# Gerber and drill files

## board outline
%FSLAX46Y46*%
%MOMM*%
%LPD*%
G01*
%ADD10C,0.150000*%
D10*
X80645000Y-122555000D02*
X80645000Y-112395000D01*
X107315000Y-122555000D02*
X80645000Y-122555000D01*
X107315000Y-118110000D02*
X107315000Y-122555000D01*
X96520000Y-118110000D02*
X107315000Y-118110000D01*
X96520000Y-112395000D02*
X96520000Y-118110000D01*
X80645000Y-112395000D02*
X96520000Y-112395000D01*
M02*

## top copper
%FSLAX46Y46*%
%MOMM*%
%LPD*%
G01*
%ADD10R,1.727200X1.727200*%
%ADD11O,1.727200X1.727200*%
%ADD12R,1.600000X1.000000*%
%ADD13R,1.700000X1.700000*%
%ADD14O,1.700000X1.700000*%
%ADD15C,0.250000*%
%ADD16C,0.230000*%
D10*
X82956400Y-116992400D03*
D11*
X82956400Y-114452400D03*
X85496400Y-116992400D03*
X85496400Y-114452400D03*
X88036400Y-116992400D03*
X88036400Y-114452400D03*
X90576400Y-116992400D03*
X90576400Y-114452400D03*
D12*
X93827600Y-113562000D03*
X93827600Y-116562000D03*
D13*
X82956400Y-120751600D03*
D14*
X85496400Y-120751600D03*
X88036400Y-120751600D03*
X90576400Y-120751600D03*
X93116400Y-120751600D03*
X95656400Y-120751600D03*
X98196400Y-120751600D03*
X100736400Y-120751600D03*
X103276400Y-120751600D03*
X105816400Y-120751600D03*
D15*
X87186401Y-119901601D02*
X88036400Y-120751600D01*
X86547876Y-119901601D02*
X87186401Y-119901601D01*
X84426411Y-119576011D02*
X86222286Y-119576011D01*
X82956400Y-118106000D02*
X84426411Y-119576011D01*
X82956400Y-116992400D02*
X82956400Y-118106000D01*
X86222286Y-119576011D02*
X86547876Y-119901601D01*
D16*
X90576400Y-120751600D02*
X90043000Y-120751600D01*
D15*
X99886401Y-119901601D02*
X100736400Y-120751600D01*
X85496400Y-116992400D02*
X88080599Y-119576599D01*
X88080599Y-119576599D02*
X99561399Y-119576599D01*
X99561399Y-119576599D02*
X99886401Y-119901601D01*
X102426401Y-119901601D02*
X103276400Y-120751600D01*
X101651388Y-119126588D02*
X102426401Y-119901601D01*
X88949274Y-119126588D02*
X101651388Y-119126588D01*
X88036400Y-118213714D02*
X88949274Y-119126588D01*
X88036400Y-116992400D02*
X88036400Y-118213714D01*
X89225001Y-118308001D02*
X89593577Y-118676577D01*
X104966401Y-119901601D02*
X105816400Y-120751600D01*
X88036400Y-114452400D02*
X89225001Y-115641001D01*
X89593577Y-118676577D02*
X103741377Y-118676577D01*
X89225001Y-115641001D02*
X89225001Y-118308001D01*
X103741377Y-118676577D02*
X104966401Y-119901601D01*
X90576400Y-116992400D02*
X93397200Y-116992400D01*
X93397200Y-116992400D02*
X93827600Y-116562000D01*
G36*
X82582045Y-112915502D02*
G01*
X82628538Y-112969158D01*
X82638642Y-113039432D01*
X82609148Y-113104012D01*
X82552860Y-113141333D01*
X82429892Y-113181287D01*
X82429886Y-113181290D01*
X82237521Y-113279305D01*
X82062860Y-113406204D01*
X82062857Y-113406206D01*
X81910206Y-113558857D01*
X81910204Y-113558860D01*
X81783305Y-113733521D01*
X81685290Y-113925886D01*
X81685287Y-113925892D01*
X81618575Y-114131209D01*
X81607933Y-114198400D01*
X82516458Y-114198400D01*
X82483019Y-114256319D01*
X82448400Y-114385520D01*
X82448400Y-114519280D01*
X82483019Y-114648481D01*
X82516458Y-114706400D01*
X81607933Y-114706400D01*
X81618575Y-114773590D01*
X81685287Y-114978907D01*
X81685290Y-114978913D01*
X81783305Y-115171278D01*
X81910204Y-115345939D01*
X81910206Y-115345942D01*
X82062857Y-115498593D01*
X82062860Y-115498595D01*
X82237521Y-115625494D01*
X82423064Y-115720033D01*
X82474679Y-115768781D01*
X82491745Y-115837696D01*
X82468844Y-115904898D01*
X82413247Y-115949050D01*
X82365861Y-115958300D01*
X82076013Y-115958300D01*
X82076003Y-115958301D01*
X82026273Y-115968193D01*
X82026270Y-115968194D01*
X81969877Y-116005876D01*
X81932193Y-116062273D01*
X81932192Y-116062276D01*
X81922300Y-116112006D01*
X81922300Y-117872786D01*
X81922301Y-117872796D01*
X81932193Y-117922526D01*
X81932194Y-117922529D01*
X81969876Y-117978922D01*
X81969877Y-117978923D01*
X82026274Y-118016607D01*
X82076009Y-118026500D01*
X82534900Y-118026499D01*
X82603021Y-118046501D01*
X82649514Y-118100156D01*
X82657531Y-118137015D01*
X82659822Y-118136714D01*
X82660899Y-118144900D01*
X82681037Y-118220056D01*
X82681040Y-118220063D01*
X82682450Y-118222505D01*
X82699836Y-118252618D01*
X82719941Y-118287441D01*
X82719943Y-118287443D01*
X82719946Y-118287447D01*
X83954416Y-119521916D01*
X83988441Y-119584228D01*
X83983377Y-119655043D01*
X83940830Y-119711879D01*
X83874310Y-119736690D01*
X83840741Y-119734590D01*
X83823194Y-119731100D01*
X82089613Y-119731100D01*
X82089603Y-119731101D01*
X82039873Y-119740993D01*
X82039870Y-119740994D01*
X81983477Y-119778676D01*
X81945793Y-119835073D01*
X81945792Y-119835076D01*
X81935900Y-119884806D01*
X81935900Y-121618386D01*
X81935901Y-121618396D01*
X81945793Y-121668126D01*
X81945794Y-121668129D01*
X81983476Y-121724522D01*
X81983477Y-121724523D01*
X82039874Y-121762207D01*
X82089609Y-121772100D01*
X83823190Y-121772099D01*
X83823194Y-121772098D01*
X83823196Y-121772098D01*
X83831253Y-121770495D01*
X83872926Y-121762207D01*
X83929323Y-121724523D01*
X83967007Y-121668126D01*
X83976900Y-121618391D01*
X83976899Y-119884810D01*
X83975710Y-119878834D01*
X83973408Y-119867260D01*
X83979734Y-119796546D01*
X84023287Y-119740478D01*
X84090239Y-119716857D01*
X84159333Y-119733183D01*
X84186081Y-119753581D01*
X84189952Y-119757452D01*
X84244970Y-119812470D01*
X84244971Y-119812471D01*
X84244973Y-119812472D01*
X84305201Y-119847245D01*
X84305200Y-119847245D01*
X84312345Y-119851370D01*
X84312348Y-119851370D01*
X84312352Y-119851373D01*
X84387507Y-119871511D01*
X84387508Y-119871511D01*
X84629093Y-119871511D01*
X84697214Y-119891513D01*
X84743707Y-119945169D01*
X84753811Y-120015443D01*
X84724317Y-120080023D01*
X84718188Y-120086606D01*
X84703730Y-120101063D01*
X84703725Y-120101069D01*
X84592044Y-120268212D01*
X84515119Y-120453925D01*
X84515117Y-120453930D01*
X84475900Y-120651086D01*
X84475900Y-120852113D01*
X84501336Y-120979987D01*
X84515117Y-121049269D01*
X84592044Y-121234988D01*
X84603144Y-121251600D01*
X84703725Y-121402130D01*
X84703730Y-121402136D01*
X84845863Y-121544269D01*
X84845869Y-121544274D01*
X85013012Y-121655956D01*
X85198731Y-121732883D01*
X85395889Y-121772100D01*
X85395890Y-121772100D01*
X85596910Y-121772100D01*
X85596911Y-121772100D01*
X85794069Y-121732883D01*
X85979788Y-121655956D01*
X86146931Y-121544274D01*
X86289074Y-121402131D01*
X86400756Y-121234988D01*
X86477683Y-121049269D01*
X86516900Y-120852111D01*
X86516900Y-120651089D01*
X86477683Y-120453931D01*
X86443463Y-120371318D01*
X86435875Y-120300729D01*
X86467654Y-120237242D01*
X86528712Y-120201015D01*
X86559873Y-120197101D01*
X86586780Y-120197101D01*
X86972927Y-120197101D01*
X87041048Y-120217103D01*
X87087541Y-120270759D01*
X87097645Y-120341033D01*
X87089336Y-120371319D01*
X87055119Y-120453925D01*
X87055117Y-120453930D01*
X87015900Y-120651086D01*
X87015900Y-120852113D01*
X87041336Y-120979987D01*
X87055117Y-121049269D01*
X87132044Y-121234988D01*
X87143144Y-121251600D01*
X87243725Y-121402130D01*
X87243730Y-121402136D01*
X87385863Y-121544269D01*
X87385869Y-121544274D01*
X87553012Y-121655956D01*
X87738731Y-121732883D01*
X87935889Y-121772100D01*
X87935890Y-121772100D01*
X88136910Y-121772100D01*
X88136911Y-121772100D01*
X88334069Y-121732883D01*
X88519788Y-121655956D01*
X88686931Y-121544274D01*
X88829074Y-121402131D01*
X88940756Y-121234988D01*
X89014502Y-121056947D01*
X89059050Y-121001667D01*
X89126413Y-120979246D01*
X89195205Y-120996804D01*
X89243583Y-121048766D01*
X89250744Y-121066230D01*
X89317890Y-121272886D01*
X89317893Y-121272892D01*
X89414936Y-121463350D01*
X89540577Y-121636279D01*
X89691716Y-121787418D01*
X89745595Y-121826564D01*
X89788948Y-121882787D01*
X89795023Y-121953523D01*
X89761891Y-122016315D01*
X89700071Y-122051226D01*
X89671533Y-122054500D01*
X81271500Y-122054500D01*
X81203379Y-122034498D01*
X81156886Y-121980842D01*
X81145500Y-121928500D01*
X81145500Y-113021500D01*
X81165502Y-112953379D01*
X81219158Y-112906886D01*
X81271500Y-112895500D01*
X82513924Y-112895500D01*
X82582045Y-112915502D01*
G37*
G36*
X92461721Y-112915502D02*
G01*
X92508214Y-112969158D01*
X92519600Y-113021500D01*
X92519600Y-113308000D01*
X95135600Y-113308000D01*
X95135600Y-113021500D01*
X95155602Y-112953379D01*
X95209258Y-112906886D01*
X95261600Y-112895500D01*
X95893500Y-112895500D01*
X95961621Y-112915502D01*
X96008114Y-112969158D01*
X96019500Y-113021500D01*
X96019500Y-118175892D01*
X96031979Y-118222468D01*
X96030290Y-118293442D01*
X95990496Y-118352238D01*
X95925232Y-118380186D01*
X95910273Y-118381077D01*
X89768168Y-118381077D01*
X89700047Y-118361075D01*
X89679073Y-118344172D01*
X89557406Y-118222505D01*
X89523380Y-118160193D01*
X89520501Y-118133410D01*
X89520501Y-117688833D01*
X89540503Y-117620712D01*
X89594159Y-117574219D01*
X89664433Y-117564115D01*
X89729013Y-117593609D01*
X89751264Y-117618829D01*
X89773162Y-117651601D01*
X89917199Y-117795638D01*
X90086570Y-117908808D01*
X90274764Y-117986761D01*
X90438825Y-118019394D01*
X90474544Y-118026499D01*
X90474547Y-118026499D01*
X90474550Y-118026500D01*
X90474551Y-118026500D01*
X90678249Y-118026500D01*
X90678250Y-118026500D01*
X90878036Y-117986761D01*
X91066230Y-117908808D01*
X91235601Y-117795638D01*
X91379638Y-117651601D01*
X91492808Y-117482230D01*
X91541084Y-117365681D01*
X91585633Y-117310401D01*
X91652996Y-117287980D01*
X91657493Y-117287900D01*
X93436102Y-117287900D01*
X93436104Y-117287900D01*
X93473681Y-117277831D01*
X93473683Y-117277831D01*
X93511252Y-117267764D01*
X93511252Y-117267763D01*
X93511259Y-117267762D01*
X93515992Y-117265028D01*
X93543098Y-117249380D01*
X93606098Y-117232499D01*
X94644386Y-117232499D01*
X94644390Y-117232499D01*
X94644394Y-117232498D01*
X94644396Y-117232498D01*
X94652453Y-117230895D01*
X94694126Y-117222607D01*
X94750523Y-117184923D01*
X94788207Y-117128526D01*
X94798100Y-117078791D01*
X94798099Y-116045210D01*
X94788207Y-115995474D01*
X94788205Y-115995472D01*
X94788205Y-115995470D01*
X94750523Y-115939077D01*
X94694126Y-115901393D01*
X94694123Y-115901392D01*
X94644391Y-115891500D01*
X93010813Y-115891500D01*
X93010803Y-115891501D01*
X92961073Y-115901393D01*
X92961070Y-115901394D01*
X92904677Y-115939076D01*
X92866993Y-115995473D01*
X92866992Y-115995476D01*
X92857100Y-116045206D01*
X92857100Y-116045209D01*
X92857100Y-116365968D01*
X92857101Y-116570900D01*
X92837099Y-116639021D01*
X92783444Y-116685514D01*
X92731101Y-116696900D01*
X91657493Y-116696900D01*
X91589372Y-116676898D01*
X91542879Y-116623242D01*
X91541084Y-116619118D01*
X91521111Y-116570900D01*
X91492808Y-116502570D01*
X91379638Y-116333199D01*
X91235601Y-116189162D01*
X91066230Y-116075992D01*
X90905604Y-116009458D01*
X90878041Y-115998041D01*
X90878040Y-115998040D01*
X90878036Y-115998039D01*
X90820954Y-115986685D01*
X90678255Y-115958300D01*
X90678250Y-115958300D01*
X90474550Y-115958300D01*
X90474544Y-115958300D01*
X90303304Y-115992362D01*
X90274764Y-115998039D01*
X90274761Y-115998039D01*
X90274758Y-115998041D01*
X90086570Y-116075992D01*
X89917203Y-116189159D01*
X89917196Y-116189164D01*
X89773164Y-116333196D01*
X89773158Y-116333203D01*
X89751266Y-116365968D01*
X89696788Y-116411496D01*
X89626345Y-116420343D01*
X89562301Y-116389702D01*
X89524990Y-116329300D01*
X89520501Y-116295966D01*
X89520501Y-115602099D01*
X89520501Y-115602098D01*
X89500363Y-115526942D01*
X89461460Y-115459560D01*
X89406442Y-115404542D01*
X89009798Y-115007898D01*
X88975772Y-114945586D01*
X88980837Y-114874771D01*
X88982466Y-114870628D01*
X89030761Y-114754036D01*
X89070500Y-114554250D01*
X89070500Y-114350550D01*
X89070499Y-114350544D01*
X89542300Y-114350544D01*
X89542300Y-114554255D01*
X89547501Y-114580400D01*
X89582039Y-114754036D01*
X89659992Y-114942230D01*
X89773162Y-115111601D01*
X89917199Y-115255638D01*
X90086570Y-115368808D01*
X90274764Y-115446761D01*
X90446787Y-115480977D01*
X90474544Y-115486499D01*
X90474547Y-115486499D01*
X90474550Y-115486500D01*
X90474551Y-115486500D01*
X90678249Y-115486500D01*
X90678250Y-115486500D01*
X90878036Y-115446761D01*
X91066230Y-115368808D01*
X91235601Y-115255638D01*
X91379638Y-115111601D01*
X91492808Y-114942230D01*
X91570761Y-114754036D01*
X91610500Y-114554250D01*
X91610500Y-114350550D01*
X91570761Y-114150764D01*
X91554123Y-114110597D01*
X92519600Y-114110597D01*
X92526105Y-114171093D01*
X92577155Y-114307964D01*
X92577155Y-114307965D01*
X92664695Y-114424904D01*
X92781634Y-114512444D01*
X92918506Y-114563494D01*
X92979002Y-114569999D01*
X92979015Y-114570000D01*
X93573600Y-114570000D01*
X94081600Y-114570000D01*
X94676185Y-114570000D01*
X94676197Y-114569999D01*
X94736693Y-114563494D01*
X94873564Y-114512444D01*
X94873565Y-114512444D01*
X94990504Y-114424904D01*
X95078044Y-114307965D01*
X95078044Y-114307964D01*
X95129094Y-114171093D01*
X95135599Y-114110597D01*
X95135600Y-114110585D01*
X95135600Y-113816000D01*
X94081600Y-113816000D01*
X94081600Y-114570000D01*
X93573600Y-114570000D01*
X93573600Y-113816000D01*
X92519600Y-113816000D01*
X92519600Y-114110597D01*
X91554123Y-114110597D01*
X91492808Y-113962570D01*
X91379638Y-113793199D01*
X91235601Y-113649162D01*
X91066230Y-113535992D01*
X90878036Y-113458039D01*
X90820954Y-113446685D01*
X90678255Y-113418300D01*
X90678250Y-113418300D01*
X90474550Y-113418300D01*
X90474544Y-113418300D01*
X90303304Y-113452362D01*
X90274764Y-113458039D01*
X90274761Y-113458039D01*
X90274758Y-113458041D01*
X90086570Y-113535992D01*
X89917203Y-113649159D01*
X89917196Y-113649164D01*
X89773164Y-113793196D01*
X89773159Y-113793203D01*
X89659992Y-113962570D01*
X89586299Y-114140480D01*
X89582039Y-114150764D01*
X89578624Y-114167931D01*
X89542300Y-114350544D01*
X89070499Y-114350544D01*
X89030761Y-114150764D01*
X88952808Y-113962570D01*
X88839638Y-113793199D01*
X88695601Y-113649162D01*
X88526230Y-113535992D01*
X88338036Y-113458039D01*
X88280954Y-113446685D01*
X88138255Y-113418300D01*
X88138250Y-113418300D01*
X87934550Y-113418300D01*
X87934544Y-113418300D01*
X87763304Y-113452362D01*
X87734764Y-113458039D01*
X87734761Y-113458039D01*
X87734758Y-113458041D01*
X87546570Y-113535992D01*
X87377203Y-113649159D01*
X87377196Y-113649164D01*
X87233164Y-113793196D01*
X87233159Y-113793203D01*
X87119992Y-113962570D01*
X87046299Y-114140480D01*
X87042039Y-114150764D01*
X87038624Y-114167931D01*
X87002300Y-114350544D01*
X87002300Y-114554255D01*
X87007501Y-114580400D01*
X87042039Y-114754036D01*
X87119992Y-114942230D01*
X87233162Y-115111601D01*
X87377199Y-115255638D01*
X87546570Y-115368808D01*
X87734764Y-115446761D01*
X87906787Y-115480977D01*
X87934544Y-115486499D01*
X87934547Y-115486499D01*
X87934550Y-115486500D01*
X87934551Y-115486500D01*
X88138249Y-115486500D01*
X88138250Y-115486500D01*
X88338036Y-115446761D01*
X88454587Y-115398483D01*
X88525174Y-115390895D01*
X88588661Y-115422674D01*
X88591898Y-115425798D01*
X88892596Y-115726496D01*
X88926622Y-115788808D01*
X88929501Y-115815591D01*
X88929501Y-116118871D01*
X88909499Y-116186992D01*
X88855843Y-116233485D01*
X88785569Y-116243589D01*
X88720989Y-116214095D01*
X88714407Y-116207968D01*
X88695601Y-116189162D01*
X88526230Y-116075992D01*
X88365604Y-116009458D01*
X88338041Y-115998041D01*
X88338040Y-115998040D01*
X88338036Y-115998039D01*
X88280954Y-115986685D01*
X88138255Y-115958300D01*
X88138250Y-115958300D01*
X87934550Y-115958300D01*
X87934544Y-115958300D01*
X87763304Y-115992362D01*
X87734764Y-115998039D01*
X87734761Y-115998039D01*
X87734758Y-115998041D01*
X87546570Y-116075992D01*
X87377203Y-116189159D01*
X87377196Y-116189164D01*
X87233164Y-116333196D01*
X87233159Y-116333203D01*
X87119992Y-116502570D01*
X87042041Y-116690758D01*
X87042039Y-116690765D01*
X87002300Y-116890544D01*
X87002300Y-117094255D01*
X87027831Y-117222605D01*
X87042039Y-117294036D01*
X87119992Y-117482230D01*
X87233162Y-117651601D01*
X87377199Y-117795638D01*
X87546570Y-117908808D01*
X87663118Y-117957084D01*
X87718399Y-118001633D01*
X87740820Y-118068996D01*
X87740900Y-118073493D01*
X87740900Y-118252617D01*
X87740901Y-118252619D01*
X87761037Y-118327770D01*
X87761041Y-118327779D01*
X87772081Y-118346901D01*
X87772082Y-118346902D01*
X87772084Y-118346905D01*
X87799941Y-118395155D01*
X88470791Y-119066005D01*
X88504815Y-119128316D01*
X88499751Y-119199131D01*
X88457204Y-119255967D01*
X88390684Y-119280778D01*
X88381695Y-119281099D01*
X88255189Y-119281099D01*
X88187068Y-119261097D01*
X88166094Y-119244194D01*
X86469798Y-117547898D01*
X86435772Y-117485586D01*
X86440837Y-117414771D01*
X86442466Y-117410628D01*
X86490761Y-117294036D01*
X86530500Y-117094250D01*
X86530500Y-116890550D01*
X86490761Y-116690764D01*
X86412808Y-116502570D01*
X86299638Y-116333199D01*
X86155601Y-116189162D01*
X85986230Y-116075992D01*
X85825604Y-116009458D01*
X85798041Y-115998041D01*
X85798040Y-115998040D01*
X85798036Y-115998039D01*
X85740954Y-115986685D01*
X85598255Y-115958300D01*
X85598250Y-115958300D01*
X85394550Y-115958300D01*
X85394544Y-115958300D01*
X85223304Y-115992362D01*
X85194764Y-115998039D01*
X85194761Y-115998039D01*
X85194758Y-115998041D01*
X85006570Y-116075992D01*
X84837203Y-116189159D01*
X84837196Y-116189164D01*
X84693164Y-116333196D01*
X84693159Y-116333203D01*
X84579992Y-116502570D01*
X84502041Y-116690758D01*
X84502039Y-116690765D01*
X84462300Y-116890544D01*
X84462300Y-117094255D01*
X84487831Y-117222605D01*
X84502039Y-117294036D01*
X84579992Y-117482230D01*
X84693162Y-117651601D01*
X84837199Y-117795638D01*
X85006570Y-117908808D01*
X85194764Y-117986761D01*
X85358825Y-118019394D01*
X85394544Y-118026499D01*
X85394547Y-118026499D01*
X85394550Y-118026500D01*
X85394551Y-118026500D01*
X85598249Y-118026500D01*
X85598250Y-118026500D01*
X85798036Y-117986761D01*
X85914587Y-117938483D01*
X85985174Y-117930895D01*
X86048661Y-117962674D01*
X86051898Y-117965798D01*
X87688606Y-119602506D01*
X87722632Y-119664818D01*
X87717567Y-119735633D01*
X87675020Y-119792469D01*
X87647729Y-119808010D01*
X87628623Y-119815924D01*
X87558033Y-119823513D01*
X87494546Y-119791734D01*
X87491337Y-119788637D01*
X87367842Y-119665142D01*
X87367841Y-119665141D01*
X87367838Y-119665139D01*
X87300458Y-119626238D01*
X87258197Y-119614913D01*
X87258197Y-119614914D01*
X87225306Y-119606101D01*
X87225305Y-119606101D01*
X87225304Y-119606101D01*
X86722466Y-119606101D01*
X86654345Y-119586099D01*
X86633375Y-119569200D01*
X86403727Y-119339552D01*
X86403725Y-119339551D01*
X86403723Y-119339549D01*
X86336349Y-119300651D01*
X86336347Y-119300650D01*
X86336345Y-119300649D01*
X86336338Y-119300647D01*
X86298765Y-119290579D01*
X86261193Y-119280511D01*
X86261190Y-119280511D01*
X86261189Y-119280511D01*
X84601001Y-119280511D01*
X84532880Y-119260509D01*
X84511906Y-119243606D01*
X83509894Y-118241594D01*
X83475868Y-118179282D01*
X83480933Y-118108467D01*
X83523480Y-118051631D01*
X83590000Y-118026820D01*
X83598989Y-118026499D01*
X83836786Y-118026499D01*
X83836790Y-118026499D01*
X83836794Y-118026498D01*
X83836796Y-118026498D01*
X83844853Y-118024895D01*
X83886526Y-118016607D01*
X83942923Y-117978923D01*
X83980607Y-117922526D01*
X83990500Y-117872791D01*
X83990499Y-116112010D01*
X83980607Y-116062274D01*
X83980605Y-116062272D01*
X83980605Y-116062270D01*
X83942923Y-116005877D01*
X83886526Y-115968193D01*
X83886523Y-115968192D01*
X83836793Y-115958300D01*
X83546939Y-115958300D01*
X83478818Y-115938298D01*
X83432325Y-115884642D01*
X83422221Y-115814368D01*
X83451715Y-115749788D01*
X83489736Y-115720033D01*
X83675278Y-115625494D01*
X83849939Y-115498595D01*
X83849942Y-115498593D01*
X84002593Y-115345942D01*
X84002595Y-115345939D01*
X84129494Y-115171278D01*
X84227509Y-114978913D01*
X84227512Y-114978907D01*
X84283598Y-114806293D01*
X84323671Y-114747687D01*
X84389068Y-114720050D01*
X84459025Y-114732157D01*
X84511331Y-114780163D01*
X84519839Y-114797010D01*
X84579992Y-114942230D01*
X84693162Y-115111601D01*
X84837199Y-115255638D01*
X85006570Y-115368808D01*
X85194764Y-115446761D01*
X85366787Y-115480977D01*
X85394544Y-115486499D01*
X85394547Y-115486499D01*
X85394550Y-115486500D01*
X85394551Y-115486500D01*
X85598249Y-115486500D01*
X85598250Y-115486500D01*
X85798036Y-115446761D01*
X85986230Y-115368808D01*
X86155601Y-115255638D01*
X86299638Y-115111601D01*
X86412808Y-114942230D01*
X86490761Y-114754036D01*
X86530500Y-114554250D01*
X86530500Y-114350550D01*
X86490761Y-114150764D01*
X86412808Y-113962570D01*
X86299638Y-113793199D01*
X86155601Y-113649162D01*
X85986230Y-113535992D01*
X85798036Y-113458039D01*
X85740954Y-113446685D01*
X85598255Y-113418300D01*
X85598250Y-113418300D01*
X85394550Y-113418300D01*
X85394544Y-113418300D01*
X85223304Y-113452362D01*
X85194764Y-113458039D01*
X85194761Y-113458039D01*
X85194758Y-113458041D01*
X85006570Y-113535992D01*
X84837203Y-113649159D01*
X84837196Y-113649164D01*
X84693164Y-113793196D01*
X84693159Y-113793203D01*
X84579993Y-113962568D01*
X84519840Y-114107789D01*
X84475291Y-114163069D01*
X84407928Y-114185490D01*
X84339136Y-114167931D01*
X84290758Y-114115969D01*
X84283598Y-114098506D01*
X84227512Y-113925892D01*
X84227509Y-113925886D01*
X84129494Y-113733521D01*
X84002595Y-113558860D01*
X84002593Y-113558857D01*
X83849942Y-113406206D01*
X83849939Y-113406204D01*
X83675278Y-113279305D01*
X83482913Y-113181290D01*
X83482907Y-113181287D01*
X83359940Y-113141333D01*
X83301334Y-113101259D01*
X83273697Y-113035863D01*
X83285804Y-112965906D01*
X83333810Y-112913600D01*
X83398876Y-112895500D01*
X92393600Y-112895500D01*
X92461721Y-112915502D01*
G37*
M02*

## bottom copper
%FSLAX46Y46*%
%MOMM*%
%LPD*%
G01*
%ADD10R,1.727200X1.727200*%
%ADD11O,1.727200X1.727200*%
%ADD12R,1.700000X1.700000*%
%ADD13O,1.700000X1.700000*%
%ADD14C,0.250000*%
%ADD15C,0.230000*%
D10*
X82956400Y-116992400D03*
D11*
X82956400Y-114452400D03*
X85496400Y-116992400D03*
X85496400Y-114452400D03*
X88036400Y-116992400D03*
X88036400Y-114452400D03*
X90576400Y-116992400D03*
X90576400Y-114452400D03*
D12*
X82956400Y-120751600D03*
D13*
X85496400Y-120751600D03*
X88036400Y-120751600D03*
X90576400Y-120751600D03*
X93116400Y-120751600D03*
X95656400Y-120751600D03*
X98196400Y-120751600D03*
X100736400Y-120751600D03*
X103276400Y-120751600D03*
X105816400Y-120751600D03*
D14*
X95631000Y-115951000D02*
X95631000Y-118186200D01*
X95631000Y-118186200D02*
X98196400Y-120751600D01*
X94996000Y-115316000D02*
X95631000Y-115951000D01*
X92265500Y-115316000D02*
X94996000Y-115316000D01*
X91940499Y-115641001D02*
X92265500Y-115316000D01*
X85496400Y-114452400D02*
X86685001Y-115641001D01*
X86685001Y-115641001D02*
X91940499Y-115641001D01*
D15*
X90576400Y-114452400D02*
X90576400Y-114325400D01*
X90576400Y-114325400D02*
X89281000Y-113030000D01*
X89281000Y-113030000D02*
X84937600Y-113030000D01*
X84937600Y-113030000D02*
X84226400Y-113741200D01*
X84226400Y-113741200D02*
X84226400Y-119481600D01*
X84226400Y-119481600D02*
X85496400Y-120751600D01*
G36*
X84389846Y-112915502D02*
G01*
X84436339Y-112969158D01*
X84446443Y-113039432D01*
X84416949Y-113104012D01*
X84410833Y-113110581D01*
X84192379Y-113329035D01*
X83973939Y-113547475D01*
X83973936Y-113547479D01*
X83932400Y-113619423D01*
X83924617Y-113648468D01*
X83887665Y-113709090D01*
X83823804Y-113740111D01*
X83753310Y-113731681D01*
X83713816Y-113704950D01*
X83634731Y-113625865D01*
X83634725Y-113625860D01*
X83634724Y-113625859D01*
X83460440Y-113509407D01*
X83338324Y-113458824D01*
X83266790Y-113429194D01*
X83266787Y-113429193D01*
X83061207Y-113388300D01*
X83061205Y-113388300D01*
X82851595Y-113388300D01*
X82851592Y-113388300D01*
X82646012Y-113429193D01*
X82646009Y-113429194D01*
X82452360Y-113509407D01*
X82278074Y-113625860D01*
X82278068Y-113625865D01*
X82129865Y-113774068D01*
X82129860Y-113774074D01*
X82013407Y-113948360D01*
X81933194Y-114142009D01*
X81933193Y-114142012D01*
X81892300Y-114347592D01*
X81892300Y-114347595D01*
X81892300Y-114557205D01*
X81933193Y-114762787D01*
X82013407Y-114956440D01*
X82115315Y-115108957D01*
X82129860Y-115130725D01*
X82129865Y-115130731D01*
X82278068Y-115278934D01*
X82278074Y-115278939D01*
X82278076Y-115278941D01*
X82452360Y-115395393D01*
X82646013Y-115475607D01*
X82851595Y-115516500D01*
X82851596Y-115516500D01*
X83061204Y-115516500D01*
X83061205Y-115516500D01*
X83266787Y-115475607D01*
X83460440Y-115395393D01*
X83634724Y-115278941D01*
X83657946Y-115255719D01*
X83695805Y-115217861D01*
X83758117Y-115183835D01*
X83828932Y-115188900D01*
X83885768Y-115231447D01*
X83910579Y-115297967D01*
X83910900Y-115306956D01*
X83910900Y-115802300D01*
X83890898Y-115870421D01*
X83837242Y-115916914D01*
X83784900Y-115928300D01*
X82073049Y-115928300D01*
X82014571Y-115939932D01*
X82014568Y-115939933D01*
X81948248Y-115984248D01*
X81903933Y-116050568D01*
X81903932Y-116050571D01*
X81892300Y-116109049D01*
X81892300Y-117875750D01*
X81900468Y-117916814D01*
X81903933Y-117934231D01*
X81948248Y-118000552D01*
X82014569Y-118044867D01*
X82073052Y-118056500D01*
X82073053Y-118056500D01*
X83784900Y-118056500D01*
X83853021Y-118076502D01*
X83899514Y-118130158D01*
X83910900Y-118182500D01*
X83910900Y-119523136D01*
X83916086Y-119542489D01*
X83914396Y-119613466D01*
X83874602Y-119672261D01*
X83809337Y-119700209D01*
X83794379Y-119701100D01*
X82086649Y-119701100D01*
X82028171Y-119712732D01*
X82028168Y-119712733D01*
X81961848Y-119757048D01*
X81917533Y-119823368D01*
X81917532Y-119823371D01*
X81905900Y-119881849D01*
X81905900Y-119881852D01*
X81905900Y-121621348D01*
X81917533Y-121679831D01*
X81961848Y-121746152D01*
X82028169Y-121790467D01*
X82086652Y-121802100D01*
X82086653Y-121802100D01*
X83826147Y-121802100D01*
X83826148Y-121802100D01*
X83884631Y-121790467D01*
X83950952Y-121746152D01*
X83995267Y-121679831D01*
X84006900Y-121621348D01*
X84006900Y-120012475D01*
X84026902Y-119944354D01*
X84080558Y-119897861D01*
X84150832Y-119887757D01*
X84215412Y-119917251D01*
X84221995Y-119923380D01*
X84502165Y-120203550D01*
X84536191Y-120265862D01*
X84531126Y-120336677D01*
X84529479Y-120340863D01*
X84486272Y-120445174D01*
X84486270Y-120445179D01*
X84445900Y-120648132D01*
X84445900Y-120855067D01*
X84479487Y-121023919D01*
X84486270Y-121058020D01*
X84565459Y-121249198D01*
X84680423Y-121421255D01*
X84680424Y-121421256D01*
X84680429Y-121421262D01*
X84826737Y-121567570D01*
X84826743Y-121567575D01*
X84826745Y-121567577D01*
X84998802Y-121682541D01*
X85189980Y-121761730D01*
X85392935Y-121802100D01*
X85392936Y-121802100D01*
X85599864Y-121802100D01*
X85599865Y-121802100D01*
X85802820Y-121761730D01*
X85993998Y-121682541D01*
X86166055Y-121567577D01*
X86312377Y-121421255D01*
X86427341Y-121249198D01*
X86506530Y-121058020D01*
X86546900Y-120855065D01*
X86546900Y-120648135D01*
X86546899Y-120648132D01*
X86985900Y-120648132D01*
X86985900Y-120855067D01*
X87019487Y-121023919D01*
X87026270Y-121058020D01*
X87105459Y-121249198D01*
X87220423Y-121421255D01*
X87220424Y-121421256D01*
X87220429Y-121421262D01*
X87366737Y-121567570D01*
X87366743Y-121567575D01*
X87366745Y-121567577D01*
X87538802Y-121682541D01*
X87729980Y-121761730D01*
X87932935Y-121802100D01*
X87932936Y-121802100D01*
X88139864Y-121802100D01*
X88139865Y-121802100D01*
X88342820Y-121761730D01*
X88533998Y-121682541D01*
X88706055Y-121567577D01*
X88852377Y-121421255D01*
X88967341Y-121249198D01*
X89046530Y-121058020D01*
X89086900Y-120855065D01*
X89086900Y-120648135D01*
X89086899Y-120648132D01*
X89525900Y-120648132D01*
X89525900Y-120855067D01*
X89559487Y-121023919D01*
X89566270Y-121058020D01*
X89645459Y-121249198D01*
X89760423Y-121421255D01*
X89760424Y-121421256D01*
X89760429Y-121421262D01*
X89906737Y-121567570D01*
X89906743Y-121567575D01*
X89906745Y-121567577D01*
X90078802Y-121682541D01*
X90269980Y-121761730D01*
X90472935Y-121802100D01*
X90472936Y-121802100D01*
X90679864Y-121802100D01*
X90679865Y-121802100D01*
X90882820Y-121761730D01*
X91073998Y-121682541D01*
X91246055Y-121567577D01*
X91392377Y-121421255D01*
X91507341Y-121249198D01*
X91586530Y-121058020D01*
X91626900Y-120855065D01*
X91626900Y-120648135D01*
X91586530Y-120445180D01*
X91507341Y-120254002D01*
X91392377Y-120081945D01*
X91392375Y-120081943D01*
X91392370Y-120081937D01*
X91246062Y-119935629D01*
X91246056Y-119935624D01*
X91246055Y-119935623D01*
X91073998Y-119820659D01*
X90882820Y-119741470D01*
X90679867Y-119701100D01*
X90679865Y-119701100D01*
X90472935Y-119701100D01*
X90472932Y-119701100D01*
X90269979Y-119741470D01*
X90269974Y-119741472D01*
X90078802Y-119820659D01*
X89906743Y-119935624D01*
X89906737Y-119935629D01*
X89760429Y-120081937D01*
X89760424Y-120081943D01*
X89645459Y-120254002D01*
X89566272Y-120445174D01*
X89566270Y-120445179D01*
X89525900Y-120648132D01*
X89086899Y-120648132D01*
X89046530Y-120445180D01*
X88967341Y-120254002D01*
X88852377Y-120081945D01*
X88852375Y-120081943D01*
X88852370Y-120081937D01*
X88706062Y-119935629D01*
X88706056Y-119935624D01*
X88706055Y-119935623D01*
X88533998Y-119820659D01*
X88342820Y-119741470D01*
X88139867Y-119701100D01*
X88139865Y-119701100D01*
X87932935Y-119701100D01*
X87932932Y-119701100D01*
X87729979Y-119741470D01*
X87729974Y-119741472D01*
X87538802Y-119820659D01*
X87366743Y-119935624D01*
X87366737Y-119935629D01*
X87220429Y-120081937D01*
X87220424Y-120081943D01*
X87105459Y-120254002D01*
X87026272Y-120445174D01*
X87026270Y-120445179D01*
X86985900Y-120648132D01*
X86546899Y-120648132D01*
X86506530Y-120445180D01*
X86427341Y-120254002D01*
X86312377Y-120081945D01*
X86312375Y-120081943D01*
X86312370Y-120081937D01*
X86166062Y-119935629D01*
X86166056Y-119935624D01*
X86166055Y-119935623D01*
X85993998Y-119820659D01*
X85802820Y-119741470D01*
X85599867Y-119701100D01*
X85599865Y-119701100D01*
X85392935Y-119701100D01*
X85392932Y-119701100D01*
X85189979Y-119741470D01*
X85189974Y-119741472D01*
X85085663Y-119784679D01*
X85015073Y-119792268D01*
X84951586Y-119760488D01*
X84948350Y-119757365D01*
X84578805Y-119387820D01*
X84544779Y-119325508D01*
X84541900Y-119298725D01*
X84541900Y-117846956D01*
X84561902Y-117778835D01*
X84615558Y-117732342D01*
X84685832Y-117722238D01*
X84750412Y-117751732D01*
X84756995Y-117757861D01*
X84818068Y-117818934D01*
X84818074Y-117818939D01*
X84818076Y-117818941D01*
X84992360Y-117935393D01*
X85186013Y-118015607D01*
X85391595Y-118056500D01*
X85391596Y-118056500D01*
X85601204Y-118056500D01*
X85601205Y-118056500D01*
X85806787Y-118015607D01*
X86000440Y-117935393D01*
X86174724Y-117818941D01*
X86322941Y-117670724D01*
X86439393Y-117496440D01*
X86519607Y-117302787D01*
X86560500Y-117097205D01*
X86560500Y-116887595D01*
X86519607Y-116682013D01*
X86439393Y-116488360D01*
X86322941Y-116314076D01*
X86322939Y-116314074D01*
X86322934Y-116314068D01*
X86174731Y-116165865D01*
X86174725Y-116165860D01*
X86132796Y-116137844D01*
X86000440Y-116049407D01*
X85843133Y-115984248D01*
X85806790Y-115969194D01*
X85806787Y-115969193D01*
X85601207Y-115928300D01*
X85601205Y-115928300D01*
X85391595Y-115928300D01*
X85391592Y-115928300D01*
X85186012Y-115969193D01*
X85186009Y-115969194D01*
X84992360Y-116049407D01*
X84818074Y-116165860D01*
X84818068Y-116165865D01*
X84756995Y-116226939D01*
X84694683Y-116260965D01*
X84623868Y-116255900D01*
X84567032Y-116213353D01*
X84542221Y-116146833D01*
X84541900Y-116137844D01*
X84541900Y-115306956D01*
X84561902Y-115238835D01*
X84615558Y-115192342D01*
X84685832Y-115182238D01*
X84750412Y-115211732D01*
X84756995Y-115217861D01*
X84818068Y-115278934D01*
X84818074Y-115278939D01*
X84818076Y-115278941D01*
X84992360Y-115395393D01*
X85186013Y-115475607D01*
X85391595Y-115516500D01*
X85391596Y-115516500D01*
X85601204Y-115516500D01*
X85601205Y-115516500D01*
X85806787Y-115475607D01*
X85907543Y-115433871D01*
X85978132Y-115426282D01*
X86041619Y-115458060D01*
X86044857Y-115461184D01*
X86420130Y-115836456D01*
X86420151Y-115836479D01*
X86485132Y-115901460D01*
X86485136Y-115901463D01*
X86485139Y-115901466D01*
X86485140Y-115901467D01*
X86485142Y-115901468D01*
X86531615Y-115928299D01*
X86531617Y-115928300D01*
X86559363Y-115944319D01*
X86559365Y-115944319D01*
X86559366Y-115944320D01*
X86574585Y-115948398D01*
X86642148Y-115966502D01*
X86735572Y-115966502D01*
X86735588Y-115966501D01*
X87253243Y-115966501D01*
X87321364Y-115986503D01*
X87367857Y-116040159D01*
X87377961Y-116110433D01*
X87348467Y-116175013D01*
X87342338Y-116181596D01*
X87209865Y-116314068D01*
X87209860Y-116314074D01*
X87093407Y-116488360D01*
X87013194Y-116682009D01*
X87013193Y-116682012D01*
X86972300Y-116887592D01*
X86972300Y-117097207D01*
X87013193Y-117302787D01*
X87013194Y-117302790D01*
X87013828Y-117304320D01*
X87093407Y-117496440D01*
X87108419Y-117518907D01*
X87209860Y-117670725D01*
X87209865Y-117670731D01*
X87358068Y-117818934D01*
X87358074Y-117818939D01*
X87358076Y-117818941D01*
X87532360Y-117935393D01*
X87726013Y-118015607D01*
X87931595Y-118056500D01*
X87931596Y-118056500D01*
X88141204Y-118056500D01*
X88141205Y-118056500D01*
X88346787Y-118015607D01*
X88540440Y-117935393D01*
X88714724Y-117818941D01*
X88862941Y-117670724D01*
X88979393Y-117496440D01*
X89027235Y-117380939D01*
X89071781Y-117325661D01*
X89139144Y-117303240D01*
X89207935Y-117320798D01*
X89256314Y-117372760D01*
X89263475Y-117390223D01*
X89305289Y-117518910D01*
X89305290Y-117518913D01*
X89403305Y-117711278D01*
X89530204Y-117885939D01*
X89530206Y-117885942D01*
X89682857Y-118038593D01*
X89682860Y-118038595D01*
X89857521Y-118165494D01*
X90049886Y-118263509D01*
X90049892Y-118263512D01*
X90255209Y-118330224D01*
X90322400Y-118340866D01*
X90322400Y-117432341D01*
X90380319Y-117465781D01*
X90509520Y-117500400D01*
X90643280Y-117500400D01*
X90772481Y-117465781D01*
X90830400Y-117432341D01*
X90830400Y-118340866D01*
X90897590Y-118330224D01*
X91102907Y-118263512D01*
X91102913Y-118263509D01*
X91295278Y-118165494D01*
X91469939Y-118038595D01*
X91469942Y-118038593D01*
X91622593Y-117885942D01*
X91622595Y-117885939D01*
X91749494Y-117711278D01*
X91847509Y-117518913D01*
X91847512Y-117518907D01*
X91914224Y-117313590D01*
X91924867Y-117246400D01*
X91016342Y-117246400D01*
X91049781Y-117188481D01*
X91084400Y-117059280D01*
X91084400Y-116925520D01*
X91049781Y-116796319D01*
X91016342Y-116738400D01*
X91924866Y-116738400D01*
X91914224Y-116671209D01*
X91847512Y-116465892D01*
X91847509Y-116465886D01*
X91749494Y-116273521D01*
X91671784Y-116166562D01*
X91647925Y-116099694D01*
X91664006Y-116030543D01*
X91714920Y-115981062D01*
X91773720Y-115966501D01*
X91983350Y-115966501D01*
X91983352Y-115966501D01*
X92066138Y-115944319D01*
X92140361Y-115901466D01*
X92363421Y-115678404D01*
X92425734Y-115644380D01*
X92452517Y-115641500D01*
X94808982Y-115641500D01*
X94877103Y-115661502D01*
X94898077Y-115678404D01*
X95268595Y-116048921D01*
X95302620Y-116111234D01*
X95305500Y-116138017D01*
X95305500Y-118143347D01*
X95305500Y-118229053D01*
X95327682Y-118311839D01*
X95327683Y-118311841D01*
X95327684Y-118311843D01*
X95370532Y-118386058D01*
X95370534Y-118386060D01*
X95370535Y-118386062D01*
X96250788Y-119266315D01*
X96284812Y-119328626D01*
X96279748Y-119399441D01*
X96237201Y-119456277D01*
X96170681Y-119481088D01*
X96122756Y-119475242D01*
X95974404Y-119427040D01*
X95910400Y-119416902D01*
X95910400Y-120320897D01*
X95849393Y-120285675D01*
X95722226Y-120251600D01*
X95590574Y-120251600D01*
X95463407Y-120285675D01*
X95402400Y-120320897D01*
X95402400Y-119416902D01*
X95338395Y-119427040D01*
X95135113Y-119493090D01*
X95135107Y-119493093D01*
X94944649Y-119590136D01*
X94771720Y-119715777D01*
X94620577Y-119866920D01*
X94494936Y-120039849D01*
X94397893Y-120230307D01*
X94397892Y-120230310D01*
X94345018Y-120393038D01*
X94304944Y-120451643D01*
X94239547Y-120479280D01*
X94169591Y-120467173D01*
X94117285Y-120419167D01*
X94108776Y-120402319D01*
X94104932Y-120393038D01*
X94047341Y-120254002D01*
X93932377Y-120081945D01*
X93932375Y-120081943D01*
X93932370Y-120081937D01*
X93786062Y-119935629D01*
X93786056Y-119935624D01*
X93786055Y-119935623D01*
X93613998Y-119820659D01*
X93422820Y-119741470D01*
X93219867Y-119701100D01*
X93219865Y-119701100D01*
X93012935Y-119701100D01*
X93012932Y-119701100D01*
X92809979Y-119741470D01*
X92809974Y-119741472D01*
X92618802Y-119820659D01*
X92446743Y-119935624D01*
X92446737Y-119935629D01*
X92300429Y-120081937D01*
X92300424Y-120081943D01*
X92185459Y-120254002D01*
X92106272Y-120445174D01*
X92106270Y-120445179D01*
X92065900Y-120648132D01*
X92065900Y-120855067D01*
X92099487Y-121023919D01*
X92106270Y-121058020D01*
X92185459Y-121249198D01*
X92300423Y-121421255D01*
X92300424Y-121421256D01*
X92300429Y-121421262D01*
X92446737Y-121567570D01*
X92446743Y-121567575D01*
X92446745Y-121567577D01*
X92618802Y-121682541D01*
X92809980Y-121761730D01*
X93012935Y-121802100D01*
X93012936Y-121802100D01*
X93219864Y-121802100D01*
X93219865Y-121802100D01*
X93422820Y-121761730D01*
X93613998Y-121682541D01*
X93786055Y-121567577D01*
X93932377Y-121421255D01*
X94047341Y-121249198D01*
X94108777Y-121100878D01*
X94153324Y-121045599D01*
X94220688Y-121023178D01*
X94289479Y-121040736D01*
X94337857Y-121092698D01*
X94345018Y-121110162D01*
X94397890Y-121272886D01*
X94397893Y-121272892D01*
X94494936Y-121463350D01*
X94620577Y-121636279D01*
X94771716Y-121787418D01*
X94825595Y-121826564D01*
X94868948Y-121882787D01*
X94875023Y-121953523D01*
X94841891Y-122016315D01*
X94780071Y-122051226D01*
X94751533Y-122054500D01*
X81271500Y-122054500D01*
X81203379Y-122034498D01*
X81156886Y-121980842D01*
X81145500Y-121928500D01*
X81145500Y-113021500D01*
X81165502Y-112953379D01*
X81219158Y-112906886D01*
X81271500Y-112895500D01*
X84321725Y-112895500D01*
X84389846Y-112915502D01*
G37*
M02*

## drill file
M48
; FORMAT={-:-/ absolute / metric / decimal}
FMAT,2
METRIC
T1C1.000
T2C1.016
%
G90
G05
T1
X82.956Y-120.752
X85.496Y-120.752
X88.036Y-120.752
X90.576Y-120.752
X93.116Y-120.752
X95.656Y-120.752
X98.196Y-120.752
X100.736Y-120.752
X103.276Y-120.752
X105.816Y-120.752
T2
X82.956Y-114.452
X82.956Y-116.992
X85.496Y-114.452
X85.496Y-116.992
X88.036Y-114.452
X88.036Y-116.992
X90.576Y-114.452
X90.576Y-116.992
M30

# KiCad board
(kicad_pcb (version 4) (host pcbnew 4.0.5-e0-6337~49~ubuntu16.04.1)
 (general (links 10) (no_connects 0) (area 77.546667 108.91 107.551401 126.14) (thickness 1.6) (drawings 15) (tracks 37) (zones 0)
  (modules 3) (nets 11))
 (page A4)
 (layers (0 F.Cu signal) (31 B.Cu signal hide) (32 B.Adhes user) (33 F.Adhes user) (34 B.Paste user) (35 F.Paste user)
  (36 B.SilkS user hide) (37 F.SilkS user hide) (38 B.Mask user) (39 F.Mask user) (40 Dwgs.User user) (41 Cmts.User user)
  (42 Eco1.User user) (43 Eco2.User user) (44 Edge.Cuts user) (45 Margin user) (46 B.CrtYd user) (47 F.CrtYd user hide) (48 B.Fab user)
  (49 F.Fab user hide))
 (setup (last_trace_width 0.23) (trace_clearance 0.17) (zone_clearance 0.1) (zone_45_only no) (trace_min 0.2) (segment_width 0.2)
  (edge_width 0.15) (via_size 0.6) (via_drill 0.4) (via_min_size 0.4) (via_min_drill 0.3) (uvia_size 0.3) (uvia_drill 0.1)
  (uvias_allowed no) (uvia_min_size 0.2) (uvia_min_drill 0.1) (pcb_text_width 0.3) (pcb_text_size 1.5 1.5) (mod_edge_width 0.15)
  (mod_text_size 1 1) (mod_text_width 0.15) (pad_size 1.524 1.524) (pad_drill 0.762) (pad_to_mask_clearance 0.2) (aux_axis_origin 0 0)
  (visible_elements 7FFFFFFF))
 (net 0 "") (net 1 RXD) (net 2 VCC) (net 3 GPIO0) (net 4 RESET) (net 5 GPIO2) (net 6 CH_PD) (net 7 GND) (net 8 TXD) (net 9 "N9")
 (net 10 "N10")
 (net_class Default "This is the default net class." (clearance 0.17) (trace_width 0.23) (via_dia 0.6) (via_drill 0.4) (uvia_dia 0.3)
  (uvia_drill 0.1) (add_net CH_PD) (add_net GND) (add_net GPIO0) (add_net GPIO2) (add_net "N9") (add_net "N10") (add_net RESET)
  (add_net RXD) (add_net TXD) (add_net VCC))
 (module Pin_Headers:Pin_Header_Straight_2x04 (layer F.Cu) (at 82.9564 116.9924 90)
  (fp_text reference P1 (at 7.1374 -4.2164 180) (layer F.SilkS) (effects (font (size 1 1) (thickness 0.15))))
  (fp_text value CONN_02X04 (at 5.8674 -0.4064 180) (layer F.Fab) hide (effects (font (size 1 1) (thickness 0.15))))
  (pad 1 thru_hole rect (at 0 0 90) (size 1.7272 1.7272) (drill 1.016) (layers *.Cu *.Mask) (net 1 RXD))
  (pad 2 thru_hole oval (at 2.54 0 90) (size 1.7272 1.7272) (drill 1.016) (layers *.Cu *.Mask) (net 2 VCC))
  (pad 3 thru_hole oval (at 0 2.54 90) (size 1.7272 1.7272) (drill 1.016) (layers *.Cu *.Mask) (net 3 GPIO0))
  (pad 4 thru_hole oval (at 2.54 2.54 90) (size 1.7272 1.7272) (drill 1.016) (layers *.Cu *.Mask) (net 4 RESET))
  (pad 5 thru_hole oval (at 0 5.08 90) (size 1.7272 1.7272) (drill 1.016) (layers *.Cu *.Mask) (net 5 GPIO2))
  (pad 6 thru_hole oval (at 2.54 5.08 90) (size 1.7272 1.7272) (drill 1.016) (layers *.Cu *.Mask) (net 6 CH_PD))
  (pad 7 thru_hole oval (at 0 7.62 90) (size 1.7272 1.7272) (drill 1.016) (layers *.Cu *.Mask) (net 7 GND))
  (pad 8 thru_hole oval (at 2.54 7.62 90) (size 1.7272 1.7272) (drill 1.016) (layers *.Cu *.Mask) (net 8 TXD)))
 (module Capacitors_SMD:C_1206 (layer F.Cu) (at 93.8276 115.062 270)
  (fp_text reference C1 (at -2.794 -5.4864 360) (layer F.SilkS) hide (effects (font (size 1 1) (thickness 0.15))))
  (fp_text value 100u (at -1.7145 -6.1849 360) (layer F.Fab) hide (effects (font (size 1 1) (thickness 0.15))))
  (pad 1 smd rect (at -1.5 0 270) (size 1 1.6) (layers F.Cu F.Paste F.Mask) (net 2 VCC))
  (pad 2 smd rect (at 1.5 0 270) (size 1 1.6) (layers F.Cu F.Paste F.Mask) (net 7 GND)))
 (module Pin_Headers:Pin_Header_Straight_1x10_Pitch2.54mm (layer F.Cu) (at 82.9564 120.7516 90)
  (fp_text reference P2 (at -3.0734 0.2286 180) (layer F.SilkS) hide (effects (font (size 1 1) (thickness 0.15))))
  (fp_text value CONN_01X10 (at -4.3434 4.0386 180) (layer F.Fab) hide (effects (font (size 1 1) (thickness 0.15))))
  (pad 1 thru_hole rect (at 0 0 90) (size 1.7 1.7) (drill 1) (layers *.Cu *.Mask) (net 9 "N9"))
  (pad 2 thru_hole oval (at 0 2.54 90) (size 1.7 1.7) (drill 1) (layers *.Cu *.Mask) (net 8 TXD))
  (pad 3 thru_hole oval (at 0 5.08 90) (size 1.7 1.7) (drill 1) (layers *.Cu *.Mask) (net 1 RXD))
  (pad 4 thru_hole oval (at 0 7.62 90) (size 1.7 1.7) (drill 1) (layers *.Cu *.Mask) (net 2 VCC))
  (pad 5 thru_hole oval (at 0 10.16 90) (size 1.7 1.7) (drill 1) (layers *.Cu *.Mask) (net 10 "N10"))
  (pad 6 thru_hole oval (at 0 12.7 90) (size 1.7 1.7) (drill 1) (layers *.Cu *.Mask) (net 7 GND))
  (pad 7 thru_hole oval (at 0 15.24 90) (size 1.7 1.7) (drill 1) (layers *.Cu *.Mask) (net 4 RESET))
  (pad 8 thru_hole oval (at 0 17.78 90) (size 1.7 1.7) (drill 1) (layers *.Cu *.Mask) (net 3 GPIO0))
  (pad 9 thru_hole oval (at 0 20.32 90) (size 1.7 1.7) (drill 1) (layers *.Cu *.Mask) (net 5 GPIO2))
  (pad 10 thru_hole oval (at 0 22.86 90) (size 1.7 1.7) (drill 1) (layers *.Cu *.Mask) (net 6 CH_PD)))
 (gr_line (start 80.645 122.555) (end 80.645 112.395) (angle 90) (layer Edge.Cuts) (width 0.15))
 (gr_line (start 107.315 122.555) (end 80.645 122.555) (angle 90) (layer Edge.Cuts) (width 0.15))
 (gr_line (start 107.315 118.11) (end 107.315 122.555) (angle 90) (layer Edge.Cuts) (width 0.15))
 (gr_line (start 96.52 118.11) (end 107.315 118.11) (angle 90) (layer Edge.Cuts) (width 0.15))
 (gr_line (start 96.52 112.395) (end 96.52 118.11) (angle 90) (layer Edge.Cuts) (width 0.15))
 (gr_line (start 80.645 112.395) (end 96.52 112.395) (angle 90) (layer Edge.Cuts) (width 0.15))
 (segment (start 87.186401 119.901601) (end 88.0364 120.7516) (width 0.25) (layer F.Cu) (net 1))
 (segment (start 86.547876 119.901601) (end 87.186401 119.901601) (width 0.25) (layer F.Cu) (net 1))
 (segment (start 84.426411 119.576011) (end 86.222286 119.576011) (width 0.25) (layer F.Cu) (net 1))
 (segment (start 82.9564 118.106) (end 84.426411 119.576011) (width 0.25) (layer F.Cu) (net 1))
 (segment (start 82.9564 116.9924) (end 82.9564 118.106) (width 0.25) (layer F.Cu) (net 1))
 (segment (start 86.222286 119.576011) (end 86.547876 119.901601) (width 0.25) (layer F.Cu) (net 1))
 (segment (start 90.5764 120.7516) (end 90.043 120.7516) (width 0.23) (layer F.Cu) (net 2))
 (segment (start 99.886401 119.901601) (end 100.7364 120.7516) (width 0.25) (layer F.Cu) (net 3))
 (segment (start 85.4964 116.9924) (end 88.080599 119.576599) (width 0.25) (layer F.Cu) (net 3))
 (segment (start 88.080599 119.576599) (end 99.561399 119.576599) (width 0.25) (layer F.Cu) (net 3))
 (segment (start 99.561399 119.576599) (end 99.886401 119.901601) (width 0.25) (layer F.Cu) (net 3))
 (segment (start 95.631 115.951) (end 95.631 118.1862) (width 0.25) (layer B.Cu) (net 4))
 (segment (start 95.631 118.1862) (end 98.1964 120.7516) (width 0.25) (layer B.Cu) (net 4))
 (segment (start 94.996 115.316) (end 95.631 115.951) (width 0.25) (layer B.Cu) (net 4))
 (segment (start 92.2655 115.316) (end 94.996 115.316) (width 0.25) (layer B.Cu) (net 4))
 (segment (start 91.940499 115.641001) (end 92.2655 115.316) (width 0.25) (layer B.Cu) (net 4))
 (segment (start 85.4964 114.4524) (end 86.685001 115.641001) (width 0.25) (layer B.Cu) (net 4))
 (segment (start 86.685001 115.641001) (end 91.940499 115.641001) (width 0.25) (layer B.Cu) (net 4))
 (segment (start 102.426401 119.901601) (end 103.2764 120.7516) (width 0.25) (layer F.Cu) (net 5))
 (segment (start 101.651388 119.126588) (end 102.426401 119.901601) (width 0.25) (layer F.Cu) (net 5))
 (segment (start 88.949274 119.126588) (end 101.651388 119.126588) (width 0.25) (layer F.Cu) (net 5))
 (segment (start 88.0364 118.213714) (end 88.949274 119.126588) (width 0.25) (layer F.Cu) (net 5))
 (segment (start 88.0364 116.9924) (end 88.0364 118.213714) (width 0.25) (layer F.Cu) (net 5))
 (segment (start 89.225001 118.308001) (end 89.593577 118.676577) (width 0.25) (layer F.Cu) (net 6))
 (segment (start 104.966401 119.901601) (end 105.8164 120.7516) (width 0.25) (layer F.Cu) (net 6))
 (segment (start 88.0364 114.4524) (end 89.225001 115.641001) (width 0.25) (layer F.Cu) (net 6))
 (segment (start 89.593577 118.676577) (end 103.741377 118.676577) (width 0.25) (layer F.Cu) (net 6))
 (segment (start 89.225001 115.641001) (end 89.225001 118.308001) (width 0.25) (layer F.Cu) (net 6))
 (segment (start 103.741377 118.676577) (end 104.966401 119.901601) (width 0.25) (layer F.Cu) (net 6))
 (segment (start 90.5764 116.9924) (end 93.3972 116.9924) (width 0.25) (layer F.Cu) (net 7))
 (segment (start 93.3972 116.9924) (end 93.8276 116.562) (width 0.25) (layer F.Cu) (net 7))
 (segment (start 90.5764 114.4524) (end 90.5764 114.3254) (width 0.23) (layer B.Cu) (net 8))
 (segment (start 90.5764 114.3254) (end 89.281 113.03) (width 0.23) (layer B.Cu) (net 8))
 (segment (start 89.281 113.03) (end 84.9376 113.03) (width 0.23) (layer B.Cu) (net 8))
 (segment (start 84.9376 113.03) (end 84.2264 113.7412) (width 0.23) (layer B.Cu) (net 8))
 (segment (start 84.2264 113.7412) (end 84.2264 119.4816) (width 0.23) (layer B.Cu) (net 8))
 (segment (start 84.2264 119.4816) (end 85.4964 120.7516) (width 0.23) (layer B.Cu) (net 8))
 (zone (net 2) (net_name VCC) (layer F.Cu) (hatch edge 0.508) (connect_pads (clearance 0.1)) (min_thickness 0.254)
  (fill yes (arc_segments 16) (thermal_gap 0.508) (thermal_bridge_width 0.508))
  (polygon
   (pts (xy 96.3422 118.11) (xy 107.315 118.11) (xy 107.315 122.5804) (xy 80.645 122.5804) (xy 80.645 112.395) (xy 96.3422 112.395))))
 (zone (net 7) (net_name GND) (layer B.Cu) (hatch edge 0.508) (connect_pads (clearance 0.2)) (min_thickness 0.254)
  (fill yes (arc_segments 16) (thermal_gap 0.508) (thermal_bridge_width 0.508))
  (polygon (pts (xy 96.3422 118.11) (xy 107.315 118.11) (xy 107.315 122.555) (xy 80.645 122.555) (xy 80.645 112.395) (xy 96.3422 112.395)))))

